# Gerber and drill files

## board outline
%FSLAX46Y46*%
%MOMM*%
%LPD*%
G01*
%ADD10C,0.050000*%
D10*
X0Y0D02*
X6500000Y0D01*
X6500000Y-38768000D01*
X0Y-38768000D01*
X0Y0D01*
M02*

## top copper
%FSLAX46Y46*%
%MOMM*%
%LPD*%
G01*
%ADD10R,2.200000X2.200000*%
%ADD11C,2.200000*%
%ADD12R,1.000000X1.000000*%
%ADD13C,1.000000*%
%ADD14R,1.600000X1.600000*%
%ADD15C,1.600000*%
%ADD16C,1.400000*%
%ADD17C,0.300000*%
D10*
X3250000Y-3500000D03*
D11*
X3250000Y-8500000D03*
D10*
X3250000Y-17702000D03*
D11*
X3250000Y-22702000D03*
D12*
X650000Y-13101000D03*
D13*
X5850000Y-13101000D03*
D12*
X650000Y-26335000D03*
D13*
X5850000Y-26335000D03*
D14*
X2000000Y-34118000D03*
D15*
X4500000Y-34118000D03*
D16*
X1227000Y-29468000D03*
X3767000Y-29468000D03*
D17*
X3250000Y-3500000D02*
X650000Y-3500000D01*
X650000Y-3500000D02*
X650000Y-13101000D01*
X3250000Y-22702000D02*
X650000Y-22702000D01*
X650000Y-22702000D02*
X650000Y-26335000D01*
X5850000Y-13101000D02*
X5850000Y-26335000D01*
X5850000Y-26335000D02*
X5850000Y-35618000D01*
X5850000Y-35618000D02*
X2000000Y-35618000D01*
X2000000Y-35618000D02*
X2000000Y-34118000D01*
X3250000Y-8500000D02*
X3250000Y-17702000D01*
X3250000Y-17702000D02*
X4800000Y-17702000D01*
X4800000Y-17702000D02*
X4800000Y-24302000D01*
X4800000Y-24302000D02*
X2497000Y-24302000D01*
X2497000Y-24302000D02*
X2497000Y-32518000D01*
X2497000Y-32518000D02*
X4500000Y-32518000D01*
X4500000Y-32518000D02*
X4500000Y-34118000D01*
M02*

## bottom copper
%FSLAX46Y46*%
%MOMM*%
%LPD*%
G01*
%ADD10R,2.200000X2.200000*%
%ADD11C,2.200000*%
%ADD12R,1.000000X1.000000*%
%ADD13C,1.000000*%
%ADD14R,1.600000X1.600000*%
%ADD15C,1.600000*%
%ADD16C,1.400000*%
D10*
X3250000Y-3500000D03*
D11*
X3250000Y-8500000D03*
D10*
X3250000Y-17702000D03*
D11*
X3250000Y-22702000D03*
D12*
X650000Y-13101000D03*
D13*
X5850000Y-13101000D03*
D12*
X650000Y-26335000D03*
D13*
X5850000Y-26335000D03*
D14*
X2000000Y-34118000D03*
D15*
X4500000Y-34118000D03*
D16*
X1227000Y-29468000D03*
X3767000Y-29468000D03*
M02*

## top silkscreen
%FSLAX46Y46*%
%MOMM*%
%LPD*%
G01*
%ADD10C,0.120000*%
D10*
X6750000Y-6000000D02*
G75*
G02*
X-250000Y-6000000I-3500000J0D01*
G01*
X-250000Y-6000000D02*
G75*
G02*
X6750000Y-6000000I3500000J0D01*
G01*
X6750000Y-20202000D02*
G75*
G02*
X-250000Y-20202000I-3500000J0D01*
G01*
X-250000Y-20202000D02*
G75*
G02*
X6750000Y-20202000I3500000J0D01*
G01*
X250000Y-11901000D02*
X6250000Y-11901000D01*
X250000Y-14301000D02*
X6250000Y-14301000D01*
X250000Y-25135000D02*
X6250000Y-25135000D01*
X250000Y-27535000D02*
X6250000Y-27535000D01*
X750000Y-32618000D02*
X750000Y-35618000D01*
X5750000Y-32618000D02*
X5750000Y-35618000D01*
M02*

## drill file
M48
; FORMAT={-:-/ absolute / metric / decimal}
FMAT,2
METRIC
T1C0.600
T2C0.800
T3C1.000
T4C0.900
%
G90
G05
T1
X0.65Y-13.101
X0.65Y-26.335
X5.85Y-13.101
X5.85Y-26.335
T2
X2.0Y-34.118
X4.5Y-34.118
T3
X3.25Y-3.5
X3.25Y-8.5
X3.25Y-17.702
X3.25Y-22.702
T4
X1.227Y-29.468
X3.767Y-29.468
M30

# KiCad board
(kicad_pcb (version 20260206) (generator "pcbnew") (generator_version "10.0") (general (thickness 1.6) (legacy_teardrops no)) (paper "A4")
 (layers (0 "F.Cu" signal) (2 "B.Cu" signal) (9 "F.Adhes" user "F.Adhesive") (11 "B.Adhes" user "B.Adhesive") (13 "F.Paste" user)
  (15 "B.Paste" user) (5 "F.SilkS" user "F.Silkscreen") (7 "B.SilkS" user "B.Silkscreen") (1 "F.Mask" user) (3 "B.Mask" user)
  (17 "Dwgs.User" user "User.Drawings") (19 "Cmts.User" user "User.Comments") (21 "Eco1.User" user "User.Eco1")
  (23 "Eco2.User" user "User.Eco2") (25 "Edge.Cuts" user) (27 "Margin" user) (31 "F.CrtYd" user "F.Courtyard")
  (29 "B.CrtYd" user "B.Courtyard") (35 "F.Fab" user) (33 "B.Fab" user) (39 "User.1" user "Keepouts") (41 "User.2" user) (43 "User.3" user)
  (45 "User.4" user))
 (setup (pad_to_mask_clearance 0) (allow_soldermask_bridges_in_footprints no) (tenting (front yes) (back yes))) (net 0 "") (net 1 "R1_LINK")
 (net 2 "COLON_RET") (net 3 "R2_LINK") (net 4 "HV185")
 (gr_rect (start 0 0) (end 6.5 38.7680) (stroke (width 0.05) (type default)) (fill none) (layer "Edge.Cuts"))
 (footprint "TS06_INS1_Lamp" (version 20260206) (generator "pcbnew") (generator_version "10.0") (layer "F.Cu") (at 3.2500 6.0000)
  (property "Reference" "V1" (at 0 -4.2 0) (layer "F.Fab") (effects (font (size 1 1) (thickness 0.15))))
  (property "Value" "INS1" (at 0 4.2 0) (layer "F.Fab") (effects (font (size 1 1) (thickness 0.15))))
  (pad "1" thru_hole rect (at 0.0000 -2.5000) (size 2.2 2.2) (drill 1.0) (layers "*.Cu" "*.Mask") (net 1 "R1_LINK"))
  (pad "2" thru_hole circle (at 0.0000 2.5000) (size 2.2 2.2) (drill 1.0) (layers "*.Cu" "*.Mask") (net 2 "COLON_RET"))
  (fp_circle (center 0 0) (end 0 3.5) (stroke (width 0.12) (type solid)) (fill no) (layer "F.SilkS")))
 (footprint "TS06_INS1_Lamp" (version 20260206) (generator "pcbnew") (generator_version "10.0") (layer "F.Cu") (at 3.2500 20.2020)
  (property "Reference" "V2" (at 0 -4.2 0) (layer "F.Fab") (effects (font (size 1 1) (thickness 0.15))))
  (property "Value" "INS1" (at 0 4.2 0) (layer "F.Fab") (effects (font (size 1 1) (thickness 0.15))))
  (pad "1" thru_hole rect (at 0.0000 -2.5000) (size 2.2 2.2) (drill 1.0) (layers "*.Cu" "*.Mask") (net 2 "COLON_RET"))
  (pad "2" thru_hole circle (at 0.0000 2.5000) (size 2.2 2.2) (drill 1.0) (layers "*.Cu" "*.Mask") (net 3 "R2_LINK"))
  (fp_circle (center 0 0) (end 0 3.5) (stroke (width 0.12) (type solid)) (fill no) (layer "F.SilkS")))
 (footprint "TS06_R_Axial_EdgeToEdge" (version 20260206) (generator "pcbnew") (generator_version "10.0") (layer "F.Cu") (at 3.2500 13.1010)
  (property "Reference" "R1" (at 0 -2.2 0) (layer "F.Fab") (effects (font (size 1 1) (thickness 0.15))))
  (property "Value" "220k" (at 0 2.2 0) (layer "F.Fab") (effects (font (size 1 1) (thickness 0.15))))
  (pad "1" thru_hole rect (at -2.6000 0.0000) (size 1.0 1.0) (drill 0.6) (layers "*.Cu" "*.Mask") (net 1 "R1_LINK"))
  (pad "2" thru_hole circle (at 2.6000 0.0000) (size 1.0 1.0) (drill 0.6) (layers "*.Cu" "*.Mask") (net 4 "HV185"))
  (fp_line (start -3.0 -1.2) (end 3.0 -1.2) (stroke (width 0.12) (type solid)) (layer "F.SilkS"))
  (fp_line (start -3.0 1.2) (end 3.0 1.2) (stroke (width 0.12) (type solid)) (layer "F.SilkS")))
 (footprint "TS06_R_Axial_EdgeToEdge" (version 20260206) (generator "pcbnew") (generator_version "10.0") (layer "F.Cu") (at 3.2500 26.3350)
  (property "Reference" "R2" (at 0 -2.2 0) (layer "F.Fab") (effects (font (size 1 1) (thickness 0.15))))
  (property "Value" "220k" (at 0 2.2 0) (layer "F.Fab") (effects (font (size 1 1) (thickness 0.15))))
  (pad "1" thru_hole rect (at -2.6000 0.0000) (size 1.0 1.0) (drill 0.6) (layers "*.Cu" "*.Mask") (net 3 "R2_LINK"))
  (pad "2" thru_hole circle (at 2.6000 0.0000) (size 1.0 1.0) (drill 0.6) (layers "*.Cu" "*.Mask") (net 4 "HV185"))
  (fp_line (start -3.0 -1.2) (end 3.0 -1.2) (stroke (width 0.12) (type solid)) (layer "F.SilkS"))
  (fp_line (start -3.0 1.2) (end 3.0 1.2) (stroke (width 0.12) (type solid)) (layer "F.SilkS")))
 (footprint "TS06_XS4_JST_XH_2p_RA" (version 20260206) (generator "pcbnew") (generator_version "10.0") (layer "F.Cu") (at 3.2500 34.1180)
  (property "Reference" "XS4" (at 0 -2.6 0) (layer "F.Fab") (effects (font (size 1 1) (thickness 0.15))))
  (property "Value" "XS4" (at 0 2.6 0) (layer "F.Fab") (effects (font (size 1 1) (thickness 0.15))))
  (pad "1" thru_hole rect (at -1.2500 0.0000) (size 1.6 1.6) (drill 0.8) (layers "*.Cu" "*.Mask") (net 4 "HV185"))
  (pad "2" thru_hole circle (at 1.2500 0.0000) (size 1.6 1.6) (drill 0.8) (layers "*.Cu" "*.Mask") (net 2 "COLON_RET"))
  (fp_line (start -2.5 -1.5) (end -2.5 1.5) (stroke (width 0.12) (type solid)) (layer "F.SilkS"))
  (fp_line (start 2.5 -1.5) (end 2.5 1.5) (stroke (width 0.12) (type solid)) (layer "F.SilkS")))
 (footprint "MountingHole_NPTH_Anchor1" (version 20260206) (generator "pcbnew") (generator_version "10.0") (layer "F.Cu")
  (at 1.2270 29.4680)
  (pad "" np_thru_hole circle (at 0 0) (size 1.4 1.4) (drill 0.9) (layers "F&B.Cu" "*.Mask")))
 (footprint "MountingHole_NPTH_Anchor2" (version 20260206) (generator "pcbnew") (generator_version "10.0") (layer "F.Cu")
  (at 3.7670 29.4680)
  (pad "" np_thru_hole circle (at 0 0) (size 1.4 1.4) (drill 0.9) (layers "F&B.Cu" "*.Mask")))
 (segment (start 3.2500 3.5000) (end 0.6500 3.5000) (width 0.3) (layer "F.Cu") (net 1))
 (segment (start 0.6500 3.5000) (end 0.6500 13.1010) (width 0.3) (layer "F.Cu") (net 1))
 (segment (start 3.2500 22.7020) (end 0.6500 22.7020) (width 0.3) (layer "F.Cu") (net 3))
 (segment (start 0.6500 22.7020) (end 0.6500 26.3350) (width 0.3) (layer "F.Cu") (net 3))
 (segment (start 5.8500 13.1010) (end 5.8500 26.3350) (width 0.3) (layer "F.Cu") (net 4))
 (segment (start 5.8500 26.3350) (end 5.8500 35.6180) (width 0.3) (layer "F.Cu") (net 4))
 (segment (start 5.8500 35.6180) (end 2.0000 35.6180) (width 0.3) (layer "F.Cu") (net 4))
 (segment (start 2.0000 35.6180) (end 2.0000 34.1180) (width 0.3) (layer "F.Cu") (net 4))
 (segment (start 3.2500 8.5000) (end 3.2500 17.7020) (width 0.3) (layer "F.Cu") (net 2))
 (segment (start 3.2500 17.7020) (end 4.8000 17.7020) (width 0.3) (layer "F.Cu") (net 2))
 (segment (start 4.8000 17.7020) (end 4.8000 24.3020) (width 0.3) (layer "F.Cu") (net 2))
 (segment (start 4.8000 24.3020) (end 2.4970 24.3020) (width 0.3) (layer "F.Cu") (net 2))
 (segment (start 2.4970 24.3020) (end 2.4970 32.5180) (width 0.3) (layer "F.Cu") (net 2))
 (segment (start 2.4970 32.5180) (end 4.5000 32.5180) (width 0.3) (layer "F.Cu") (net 2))
 (segment (start 4.5000 32.5180) (end 4.5000 34.1180) (width 0.3) (layer "F.Cu") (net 2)))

